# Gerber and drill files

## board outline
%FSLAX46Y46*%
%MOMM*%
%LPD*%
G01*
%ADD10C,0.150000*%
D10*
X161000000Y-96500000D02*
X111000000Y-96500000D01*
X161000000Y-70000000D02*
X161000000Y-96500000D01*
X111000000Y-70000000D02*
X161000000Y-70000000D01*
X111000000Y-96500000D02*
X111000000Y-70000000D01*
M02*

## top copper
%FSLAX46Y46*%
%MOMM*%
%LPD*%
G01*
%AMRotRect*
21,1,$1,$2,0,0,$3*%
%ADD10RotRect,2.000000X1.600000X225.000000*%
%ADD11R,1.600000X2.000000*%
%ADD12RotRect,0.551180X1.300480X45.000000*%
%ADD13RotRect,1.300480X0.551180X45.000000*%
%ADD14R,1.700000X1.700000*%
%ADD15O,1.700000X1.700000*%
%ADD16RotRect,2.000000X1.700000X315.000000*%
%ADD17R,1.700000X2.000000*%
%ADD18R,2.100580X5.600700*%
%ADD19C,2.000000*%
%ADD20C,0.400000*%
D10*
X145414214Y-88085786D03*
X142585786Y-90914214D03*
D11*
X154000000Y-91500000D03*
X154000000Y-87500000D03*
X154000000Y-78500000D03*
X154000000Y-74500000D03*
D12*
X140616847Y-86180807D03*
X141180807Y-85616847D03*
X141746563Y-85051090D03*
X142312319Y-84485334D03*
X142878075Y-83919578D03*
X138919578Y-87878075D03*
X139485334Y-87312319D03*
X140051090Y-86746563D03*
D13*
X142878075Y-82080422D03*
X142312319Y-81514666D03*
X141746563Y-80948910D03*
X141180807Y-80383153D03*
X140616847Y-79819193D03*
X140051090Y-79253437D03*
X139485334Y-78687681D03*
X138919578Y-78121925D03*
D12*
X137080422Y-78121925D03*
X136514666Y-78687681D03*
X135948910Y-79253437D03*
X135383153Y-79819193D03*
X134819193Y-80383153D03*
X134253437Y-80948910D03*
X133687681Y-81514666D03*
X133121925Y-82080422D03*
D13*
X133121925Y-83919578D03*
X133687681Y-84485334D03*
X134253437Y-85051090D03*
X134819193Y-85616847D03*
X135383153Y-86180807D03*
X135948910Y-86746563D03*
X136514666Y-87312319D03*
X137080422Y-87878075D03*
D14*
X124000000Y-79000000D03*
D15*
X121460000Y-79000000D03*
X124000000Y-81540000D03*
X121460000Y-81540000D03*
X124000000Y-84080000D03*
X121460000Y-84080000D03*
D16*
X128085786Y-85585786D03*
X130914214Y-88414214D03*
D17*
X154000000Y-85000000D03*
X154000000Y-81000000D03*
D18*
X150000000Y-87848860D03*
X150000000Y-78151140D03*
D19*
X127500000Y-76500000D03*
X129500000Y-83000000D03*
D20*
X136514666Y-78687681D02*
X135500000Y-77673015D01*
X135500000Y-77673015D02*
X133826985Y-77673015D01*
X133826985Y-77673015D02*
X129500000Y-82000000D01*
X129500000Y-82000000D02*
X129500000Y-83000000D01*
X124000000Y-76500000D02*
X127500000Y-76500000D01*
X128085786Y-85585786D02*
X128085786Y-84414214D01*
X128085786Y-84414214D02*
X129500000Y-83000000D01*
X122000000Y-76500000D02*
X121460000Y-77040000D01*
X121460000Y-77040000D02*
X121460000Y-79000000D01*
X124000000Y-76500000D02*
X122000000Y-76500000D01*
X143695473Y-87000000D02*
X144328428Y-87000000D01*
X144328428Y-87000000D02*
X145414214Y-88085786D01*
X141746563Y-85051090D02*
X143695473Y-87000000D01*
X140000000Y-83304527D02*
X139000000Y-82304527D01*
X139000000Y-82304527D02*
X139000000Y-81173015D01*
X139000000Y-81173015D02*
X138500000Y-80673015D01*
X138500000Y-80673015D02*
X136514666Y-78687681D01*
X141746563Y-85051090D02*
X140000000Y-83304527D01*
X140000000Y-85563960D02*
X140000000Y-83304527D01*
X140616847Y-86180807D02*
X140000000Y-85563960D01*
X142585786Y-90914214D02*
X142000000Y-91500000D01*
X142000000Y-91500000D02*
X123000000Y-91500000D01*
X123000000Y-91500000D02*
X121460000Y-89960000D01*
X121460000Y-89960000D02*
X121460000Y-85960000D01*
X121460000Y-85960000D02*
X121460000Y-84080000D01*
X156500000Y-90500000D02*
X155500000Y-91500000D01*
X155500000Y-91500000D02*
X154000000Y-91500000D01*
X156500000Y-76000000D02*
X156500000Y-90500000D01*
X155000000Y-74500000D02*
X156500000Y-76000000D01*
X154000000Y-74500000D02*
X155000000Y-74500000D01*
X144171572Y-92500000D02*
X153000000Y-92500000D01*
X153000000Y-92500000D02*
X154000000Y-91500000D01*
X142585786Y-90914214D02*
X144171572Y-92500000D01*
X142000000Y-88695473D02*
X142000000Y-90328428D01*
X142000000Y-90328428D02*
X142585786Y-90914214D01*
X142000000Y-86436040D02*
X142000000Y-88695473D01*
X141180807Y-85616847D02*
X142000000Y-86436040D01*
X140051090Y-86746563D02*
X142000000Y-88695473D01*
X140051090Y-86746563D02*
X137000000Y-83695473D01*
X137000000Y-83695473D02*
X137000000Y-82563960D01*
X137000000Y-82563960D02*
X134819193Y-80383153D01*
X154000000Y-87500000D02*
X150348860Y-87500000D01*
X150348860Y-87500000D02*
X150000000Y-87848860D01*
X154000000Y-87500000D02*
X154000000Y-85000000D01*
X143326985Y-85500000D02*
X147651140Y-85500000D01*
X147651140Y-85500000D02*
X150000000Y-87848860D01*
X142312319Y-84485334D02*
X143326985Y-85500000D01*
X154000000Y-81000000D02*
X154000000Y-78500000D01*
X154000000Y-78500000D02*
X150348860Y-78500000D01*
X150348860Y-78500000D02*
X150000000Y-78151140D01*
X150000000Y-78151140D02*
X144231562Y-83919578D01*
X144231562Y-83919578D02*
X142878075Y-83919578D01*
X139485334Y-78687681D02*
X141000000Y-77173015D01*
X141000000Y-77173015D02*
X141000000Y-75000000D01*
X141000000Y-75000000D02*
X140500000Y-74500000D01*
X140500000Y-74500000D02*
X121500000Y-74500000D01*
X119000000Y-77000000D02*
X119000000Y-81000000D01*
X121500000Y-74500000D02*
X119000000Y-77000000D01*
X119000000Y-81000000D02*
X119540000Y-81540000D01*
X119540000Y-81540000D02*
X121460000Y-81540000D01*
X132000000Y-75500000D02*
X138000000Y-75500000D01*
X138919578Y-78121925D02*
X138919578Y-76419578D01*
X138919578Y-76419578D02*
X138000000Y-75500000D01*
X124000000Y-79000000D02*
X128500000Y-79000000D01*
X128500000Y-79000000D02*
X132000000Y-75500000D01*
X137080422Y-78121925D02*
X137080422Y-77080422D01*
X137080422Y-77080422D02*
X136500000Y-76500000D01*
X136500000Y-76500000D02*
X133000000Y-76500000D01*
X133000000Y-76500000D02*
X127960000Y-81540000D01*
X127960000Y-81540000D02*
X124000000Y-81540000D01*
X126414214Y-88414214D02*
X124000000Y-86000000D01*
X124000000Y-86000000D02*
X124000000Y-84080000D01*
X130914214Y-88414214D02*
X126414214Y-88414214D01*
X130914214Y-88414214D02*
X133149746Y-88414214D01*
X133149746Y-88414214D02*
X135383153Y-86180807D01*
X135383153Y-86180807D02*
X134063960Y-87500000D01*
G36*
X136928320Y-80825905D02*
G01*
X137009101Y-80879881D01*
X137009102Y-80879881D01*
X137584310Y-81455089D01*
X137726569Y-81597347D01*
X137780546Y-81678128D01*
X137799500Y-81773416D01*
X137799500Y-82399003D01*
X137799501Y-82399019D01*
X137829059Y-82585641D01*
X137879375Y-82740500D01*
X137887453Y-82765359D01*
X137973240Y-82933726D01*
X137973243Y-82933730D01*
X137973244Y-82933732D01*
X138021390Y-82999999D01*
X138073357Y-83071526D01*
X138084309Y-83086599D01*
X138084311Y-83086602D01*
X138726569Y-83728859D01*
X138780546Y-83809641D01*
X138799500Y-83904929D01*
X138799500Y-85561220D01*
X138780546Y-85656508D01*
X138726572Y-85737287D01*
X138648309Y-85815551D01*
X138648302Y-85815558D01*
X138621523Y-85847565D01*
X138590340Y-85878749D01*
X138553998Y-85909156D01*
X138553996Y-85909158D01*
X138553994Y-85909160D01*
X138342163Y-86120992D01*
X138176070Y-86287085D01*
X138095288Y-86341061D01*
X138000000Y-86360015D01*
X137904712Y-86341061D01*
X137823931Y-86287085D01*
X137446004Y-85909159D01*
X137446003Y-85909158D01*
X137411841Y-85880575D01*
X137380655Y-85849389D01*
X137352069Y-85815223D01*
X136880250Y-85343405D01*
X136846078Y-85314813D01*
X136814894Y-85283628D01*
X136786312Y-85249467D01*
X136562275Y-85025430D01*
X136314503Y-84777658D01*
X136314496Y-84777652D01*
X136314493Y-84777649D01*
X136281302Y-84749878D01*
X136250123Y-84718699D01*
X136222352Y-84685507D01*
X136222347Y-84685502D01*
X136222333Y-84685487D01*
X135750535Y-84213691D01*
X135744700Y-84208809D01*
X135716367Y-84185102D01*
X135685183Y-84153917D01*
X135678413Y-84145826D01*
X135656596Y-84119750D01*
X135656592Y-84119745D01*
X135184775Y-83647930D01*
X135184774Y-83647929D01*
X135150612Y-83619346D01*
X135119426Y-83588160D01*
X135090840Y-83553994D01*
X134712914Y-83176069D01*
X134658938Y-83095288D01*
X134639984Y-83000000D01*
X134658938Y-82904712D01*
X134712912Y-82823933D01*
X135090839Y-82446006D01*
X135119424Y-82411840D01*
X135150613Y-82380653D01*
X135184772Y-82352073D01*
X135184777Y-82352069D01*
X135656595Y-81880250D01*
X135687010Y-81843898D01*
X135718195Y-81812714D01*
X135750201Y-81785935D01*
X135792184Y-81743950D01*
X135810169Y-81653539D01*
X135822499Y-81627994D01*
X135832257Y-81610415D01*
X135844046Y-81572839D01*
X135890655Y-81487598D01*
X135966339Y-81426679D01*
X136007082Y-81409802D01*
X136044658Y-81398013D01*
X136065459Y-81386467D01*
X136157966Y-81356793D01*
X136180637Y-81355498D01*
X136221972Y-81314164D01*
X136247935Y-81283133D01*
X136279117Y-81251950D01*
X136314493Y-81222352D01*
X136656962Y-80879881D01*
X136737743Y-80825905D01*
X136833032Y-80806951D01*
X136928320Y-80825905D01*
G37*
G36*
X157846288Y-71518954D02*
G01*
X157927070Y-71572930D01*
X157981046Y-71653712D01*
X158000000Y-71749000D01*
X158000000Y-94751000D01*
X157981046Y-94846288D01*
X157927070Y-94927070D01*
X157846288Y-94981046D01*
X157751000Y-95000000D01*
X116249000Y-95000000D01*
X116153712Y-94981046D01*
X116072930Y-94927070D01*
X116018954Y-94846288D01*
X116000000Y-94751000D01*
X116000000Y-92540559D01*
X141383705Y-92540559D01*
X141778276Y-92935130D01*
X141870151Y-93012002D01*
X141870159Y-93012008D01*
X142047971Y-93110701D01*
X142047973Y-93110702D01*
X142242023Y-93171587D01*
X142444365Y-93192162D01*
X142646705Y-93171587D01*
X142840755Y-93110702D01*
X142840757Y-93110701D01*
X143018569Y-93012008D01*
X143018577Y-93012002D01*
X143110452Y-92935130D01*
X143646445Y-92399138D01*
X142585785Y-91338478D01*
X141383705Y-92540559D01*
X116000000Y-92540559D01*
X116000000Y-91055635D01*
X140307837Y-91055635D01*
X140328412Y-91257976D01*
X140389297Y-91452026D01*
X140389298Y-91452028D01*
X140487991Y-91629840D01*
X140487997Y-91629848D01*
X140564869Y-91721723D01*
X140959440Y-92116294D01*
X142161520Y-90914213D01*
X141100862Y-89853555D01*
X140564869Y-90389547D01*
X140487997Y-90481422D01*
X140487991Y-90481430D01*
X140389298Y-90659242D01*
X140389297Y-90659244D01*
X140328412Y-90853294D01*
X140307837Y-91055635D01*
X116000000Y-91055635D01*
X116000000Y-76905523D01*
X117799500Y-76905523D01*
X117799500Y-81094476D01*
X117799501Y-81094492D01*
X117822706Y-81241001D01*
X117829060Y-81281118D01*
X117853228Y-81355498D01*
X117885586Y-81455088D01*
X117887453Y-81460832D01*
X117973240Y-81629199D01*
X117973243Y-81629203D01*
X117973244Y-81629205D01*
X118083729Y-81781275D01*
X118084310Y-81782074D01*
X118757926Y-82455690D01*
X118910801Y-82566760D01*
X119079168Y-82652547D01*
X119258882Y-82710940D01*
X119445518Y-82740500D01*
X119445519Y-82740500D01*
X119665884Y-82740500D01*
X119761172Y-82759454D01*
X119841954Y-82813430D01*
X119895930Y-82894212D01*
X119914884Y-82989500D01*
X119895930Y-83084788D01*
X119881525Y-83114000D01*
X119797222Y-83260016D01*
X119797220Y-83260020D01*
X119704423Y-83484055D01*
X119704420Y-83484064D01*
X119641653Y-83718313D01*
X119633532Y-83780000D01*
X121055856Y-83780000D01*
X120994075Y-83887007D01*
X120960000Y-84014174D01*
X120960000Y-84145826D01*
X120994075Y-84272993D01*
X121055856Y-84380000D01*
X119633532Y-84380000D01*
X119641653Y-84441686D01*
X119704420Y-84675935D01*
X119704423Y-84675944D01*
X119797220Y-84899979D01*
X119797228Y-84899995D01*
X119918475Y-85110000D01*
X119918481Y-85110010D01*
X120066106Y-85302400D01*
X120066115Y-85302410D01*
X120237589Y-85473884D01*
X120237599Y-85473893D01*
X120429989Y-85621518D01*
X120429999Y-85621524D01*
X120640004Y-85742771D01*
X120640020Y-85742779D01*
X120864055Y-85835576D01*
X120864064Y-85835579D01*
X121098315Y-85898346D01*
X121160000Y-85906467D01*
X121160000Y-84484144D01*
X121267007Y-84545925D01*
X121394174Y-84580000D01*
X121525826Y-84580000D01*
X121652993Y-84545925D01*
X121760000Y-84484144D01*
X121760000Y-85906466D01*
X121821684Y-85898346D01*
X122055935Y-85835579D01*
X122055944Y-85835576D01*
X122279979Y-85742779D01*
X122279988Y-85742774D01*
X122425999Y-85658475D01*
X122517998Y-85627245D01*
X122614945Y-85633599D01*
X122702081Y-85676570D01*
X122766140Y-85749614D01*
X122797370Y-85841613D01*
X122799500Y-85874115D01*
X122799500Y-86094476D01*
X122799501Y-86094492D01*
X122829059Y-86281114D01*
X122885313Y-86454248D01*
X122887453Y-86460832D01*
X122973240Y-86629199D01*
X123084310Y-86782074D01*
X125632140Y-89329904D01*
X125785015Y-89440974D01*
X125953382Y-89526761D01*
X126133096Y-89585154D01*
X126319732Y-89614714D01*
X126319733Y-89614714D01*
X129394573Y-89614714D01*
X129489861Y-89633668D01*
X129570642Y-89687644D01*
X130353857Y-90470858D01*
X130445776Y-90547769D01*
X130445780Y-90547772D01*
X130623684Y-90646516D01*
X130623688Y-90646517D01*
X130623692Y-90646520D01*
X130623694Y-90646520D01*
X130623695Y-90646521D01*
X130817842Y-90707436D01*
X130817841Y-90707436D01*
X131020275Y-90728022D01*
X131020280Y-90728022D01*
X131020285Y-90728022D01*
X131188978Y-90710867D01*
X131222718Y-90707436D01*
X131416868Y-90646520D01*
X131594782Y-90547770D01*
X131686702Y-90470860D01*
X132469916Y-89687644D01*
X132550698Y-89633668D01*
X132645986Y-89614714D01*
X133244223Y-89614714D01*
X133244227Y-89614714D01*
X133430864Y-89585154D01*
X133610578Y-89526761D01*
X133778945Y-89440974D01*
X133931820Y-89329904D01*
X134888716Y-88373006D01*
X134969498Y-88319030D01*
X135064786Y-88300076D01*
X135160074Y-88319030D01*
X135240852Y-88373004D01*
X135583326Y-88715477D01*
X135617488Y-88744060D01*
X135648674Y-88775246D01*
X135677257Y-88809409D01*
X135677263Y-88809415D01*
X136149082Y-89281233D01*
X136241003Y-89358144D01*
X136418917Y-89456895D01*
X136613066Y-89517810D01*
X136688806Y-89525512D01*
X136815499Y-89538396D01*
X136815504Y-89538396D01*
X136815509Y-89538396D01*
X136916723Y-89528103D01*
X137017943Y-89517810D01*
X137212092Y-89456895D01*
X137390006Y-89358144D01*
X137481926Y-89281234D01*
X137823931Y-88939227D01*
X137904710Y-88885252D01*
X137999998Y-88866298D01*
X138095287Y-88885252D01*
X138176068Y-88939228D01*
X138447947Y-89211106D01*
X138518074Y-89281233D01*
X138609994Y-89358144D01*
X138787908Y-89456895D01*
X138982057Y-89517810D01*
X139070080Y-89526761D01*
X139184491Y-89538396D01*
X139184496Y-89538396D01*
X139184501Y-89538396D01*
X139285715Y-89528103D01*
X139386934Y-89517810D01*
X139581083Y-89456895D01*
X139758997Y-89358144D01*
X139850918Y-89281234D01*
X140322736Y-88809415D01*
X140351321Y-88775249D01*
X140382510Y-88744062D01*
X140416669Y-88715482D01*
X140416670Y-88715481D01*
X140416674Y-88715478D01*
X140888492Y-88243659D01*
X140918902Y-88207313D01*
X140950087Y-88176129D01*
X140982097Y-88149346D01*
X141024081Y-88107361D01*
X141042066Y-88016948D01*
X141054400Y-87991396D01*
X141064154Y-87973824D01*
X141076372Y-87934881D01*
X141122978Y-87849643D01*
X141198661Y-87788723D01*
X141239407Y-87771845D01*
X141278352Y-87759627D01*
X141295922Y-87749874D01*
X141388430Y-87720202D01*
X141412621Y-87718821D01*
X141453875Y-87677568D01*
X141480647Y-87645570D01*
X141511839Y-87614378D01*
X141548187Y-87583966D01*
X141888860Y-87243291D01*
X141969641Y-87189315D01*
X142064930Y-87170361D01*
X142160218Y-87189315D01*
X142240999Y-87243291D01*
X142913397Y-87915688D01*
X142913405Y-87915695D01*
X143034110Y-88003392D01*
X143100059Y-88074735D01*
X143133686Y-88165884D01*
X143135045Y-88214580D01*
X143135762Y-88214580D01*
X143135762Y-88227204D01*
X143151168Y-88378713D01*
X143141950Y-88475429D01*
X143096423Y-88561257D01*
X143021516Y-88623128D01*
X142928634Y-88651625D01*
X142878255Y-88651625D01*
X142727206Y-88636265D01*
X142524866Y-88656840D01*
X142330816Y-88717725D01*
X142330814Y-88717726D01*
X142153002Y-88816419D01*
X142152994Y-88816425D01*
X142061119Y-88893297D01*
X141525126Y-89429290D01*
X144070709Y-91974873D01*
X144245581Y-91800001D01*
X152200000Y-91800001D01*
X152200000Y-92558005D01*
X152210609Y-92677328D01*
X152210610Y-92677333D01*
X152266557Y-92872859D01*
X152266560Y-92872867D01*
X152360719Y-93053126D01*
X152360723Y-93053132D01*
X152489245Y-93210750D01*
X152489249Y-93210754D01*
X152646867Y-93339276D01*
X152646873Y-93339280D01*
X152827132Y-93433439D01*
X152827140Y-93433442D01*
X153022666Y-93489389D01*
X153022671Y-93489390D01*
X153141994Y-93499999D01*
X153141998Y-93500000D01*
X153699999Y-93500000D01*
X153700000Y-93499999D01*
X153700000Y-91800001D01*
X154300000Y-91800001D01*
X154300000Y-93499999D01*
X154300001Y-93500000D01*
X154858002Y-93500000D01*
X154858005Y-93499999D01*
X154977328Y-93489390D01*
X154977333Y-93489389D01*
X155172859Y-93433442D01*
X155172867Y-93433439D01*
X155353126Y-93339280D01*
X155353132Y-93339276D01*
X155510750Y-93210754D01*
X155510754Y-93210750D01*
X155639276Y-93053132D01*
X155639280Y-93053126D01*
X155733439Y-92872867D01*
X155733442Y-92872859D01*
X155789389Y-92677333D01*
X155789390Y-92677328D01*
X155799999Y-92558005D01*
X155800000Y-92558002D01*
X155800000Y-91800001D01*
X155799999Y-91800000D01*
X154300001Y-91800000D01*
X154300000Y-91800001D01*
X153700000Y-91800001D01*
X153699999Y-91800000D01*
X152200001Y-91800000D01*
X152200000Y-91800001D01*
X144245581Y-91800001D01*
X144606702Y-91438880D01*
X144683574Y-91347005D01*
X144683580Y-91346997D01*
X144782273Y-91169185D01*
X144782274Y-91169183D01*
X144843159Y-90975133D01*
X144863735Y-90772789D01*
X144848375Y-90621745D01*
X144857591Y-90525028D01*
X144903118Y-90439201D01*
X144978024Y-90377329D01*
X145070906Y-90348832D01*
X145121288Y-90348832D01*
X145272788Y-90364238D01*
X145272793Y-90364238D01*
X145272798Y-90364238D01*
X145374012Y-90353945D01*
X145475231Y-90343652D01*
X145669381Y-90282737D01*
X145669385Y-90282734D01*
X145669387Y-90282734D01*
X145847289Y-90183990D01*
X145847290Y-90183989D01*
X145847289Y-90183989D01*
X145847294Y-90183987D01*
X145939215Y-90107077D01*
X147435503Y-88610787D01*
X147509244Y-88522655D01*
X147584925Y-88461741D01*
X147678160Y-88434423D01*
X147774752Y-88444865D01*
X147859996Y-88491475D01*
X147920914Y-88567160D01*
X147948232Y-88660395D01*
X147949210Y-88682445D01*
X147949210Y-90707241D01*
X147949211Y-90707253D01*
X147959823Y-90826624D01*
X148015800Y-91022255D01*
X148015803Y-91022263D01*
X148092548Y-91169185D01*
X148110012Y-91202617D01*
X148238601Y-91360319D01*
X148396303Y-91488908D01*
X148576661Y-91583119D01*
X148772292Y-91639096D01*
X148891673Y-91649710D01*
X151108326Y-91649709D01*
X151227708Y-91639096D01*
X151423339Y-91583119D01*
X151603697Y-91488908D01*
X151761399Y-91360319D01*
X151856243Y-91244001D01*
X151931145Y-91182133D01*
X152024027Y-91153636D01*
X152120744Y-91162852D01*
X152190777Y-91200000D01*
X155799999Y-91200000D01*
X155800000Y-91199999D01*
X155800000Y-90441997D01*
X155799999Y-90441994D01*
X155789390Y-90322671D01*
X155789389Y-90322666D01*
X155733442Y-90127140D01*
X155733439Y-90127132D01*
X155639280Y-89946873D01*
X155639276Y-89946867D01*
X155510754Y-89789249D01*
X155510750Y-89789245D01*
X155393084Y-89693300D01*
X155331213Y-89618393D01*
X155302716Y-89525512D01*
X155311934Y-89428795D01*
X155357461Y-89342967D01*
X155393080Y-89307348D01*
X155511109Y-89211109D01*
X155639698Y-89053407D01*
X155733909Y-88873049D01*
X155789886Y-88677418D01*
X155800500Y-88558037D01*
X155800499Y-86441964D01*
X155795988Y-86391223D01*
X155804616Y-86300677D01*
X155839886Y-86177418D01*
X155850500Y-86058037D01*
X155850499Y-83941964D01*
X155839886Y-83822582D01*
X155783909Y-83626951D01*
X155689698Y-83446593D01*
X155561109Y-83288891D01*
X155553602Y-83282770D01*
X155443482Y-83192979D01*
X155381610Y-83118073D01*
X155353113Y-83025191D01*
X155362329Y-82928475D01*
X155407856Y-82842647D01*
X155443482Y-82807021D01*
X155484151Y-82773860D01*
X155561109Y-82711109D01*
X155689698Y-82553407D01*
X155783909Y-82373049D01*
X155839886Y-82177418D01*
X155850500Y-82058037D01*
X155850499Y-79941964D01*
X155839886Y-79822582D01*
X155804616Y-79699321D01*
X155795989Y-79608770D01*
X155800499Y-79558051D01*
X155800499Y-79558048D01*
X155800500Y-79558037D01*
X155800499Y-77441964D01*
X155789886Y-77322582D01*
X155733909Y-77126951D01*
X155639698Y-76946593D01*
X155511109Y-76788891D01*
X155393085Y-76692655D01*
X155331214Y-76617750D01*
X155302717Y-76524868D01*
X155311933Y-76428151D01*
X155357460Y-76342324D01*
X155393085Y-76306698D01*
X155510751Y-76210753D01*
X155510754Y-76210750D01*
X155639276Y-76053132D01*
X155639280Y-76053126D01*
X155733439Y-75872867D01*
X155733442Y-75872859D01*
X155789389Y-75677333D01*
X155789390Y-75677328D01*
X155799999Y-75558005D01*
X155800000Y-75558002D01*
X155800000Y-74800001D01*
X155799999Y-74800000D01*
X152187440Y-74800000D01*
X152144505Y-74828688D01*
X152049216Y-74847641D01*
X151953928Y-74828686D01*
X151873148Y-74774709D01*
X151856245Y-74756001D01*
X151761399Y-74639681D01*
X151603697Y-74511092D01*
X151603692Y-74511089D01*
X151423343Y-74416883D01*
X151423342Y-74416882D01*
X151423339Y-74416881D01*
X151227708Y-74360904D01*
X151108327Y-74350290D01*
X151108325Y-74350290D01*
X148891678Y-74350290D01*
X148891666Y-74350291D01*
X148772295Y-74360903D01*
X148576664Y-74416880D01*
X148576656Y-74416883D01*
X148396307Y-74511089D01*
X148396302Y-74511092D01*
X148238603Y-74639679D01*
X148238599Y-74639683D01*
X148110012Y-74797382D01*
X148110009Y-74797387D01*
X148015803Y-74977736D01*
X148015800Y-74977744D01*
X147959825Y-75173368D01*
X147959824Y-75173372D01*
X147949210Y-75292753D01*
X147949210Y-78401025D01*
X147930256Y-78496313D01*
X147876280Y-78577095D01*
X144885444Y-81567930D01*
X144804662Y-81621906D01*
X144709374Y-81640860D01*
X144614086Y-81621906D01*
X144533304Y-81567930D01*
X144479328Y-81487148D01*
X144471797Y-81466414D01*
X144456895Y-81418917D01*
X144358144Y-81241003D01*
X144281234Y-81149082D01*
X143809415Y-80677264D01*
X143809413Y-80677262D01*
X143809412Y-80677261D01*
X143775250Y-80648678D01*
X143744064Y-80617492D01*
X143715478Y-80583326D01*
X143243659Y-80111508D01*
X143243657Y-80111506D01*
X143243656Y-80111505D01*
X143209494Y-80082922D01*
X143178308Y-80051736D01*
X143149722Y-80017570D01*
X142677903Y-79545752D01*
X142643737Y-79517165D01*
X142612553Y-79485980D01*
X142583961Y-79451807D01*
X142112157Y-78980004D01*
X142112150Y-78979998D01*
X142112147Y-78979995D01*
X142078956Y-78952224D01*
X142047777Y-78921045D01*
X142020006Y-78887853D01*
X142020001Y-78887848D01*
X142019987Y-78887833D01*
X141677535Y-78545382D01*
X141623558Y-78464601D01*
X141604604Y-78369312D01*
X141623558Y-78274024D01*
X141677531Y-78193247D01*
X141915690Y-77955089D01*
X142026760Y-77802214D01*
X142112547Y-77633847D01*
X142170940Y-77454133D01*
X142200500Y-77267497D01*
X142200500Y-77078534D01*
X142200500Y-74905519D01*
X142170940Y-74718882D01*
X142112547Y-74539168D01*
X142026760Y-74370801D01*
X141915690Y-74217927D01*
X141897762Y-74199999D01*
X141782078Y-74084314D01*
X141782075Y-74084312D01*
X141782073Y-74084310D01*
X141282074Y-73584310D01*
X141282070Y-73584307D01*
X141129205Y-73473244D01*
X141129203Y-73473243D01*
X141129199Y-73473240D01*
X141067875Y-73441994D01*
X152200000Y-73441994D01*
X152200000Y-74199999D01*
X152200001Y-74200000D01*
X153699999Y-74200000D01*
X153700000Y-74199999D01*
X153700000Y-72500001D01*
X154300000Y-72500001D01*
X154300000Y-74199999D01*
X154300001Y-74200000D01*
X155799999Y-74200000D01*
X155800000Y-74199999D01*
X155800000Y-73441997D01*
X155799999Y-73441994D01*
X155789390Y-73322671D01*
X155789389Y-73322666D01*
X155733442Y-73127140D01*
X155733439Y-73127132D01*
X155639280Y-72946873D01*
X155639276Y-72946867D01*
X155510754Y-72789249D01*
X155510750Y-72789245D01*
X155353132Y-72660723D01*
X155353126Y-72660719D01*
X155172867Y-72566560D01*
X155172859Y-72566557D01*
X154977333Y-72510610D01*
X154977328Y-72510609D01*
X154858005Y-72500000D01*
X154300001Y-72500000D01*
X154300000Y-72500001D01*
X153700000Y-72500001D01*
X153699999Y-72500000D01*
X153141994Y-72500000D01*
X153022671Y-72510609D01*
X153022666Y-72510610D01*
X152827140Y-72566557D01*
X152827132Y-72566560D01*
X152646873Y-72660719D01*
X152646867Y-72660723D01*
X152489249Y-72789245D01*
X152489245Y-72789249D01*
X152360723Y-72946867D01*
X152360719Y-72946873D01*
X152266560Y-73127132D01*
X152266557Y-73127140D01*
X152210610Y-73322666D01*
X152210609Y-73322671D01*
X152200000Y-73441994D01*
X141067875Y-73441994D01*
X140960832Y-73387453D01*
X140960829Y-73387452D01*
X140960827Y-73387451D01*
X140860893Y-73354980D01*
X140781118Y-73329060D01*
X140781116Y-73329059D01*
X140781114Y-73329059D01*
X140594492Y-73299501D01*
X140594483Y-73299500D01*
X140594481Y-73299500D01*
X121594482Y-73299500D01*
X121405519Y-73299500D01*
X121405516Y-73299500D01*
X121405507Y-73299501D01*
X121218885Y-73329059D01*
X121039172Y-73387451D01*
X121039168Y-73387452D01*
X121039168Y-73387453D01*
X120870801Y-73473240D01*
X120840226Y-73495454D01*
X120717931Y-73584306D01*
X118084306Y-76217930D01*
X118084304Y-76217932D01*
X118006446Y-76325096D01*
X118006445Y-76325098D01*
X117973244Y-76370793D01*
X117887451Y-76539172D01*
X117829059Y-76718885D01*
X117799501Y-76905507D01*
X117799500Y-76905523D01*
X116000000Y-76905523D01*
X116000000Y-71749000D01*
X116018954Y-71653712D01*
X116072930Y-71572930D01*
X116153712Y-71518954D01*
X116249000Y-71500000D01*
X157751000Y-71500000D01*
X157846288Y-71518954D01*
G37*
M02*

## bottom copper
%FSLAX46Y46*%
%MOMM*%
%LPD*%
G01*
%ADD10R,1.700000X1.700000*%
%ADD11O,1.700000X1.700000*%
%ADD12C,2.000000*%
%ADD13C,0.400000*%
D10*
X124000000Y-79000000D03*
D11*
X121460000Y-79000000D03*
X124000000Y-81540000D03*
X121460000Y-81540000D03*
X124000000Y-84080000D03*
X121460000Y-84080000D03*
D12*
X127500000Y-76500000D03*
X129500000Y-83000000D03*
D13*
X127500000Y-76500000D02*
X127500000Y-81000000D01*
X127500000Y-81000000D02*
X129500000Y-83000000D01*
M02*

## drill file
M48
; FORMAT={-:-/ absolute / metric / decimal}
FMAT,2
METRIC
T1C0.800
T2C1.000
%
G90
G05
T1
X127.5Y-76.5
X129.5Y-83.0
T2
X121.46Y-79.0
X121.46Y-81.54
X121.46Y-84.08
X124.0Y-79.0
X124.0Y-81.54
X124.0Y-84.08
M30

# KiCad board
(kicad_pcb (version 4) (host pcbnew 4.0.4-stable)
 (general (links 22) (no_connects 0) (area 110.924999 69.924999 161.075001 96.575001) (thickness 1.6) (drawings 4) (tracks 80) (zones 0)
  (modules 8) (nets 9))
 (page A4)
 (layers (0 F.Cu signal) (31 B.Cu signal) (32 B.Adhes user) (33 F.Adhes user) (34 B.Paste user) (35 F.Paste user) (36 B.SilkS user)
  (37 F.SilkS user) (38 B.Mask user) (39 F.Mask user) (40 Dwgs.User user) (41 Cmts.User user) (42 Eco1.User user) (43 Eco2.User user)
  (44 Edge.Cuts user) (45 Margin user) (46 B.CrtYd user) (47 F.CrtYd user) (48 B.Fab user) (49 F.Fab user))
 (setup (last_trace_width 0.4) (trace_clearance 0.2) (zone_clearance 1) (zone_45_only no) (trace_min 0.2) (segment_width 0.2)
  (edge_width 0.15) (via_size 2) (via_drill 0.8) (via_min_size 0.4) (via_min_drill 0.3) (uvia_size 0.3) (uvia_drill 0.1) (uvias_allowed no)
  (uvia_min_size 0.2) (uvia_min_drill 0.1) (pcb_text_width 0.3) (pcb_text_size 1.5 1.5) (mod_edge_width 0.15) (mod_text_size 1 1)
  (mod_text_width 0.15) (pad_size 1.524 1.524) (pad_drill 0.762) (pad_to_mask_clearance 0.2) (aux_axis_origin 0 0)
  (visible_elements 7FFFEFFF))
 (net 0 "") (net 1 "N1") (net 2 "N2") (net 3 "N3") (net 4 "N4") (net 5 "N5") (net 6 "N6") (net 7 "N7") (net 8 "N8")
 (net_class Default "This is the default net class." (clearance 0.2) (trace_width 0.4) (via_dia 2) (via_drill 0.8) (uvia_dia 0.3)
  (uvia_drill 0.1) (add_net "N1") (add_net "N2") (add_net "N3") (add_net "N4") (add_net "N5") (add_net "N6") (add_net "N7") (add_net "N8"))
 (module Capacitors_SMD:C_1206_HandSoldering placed (layer F.Cu) (at 144 89.5 225)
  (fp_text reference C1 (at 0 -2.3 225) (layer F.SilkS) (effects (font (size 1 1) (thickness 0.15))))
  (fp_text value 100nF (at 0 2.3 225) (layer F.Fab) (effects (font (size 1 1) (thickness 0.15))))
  (pad 1 smd rect (at -2 0 225) (size 2 1.6) (layers F.Cu F.Paste F.Mask) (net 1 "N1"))
  (pad 2 smd rect (at 2 0 225) (size 2 1.6) (layers F.Cu F.Paste F.Mask) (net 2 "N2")))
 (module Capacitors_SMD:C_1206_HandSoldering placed (layer F.Cu) (at 154 89.5 90)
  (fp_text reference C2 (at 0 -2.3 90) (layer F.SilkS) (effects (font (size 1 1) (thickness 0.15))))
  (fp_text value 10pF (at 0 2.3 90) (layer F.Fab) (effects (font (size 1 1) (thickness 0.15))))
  (pad 1 smd rect (at -2 0 90) (size 2 1.6) (layers F.Cu F.Paste F.Mask) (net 2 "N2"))
  (pad 2 smd rect (at 2 0 90) (size 2 1.6) (layers F.Cu F.Paste F.Mask) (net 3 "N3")))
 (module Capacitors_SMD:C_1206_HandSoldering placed (layer F.Cu) (at 154 76.5 90)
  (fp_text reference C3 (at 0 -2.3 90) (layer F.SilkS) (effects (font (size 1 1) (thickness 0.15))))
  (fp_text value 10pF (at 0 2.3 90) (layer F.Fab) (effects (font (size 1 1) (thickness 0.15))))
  (pad 1 smd rect (at -2 0 90) (size 2 1.6) (layers F.Cu F.Paste F.Mask) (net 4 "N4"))
  (pad 2 smd rect (at 2 0 90) (size 2 1.6) (layers F.Cu F.Paste F.Mask) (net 2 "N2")))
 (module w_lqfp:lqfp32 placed (layer F.Cu) (at 138 83 45)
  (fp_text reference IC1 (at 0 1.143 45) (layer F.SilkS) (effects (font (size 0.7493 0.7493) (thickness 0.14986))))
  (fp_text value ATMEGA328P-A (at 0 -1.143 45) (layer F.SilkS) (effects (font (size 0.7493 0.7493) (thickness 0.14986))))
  (pad 4 smd rect (at -0.39878 4.09956 45) (size 0.55118 1.30048) (layers F.Cu F.Paste F.Mask) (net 1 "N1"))
  (pad 5 smd rect (at 0.39878 4.09956 45) (size 0.55118 1.30048) (layers F.Cu F.Paste F.Mask) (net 2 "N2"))
  (pad 6 smd rect (at 1.19888 4.09956 45) (size 0.55118 1.30048) (layers F.Cu F.Paste F.Mask) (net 1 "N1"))
  (pad 7 smd rect (at 1.99898 4.09956 45) (size 0.55118 1.30048) (layers F.Cu F.Paste F.Mask) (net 3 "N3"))
  (pad 8 smd rect (at 2.79908 4.09956 45) (size 0.55118 1.30048) (layers F.Cu F.Paste F.Mask) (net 4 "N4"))
  (pad 1 smd rect (at -2.79908 4.09956 45) (size 0.55118 1.30048) (layers F.Cu F.Paste F.Mask))
  (pad 2 smd rect (at -1.99898 4.09956 45) (size 0.55118 1.30048) (layers F.Cu F.Paste F.Mask))
  (pad 3 smd rect (at -1.19888 4.09956 45) (size 0.55118 1.30048) (layers F.Cu F.Paste F.Mask) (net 2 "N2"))
  (pad 9 smd rect (at 4.09956 2.79908 45) (size 1.30048 0.55118) (layers F.Cu F.Paste F.Mask))
  (pad 10 smd rect (at 4.09956 1.99898 45) (size 1.30048 0.55118) (layers F.Cu F.Paste F.Mask))
  (pad 11 smd rect (at 4.09956 1.19888 45) (size 1.30048 0.55118) (layers F.Cu F.Paste F.Mask))
  (pad 12 smd rect (at 4.09956 0.39878 45) (size 1.30048 0.55118) (layers F.Cu F.Paste F.Mask))
  (pad 13 smd rect (at 4.09956 -0.39878 45) (size 1.30048 0.55118) (layers F.Cu F.Paste F.Mask))
  (pad 14 smd rect (at 4.09956 -1.19888 45) (size 1.30048 0.55118) (layers F.Cu F.Paste F.Mask))
  (pad 15 smd rect (at 4.09956 -1.99898 45) (size 1.30048 0.55118) (layers F.Cu F.Paste F.Mask) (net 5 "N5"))
  (pad 16 smd rect (at 4.09956 -2.79908 45) (size 1.30048 0.55118) (layers F.Cu F.Paste F.Mask) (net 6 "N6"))
  (pad 17 smd rect (at 2.79908 -4.09956 45) (size 0.55118 1.30048) (layers F.Cu F.Paste F.Mask) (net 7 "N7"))
  (pad 18 smd rect (at 1.99898 -4.09956 45) (size 0.55118 1.30048) (layers F.Cu F.Paste F.Mask) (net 1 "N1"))
  (pad 19 smd rect (at 1.19888 -4.09956 45) (size 0.55118 1.30048) (layers F.Cu F.Paste F.Mask))
  (pad 20 smd rect (at 0.39878 -4.09956 45) (size 0.55118 1.30048) (layers F.Cu F.Paste F.Mask))
  (pad 21 smd rect (at -0.39878 -4.09956 45) (size 0.55118 1.30048) (layers F.Cu F.Paste F.Mask) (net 2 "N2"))
  (pad 22 smd rect (at -1.19888 -4.09956 45) (size 0.55118 1.30048) (layers F.Cu F.Paste F.Mask))
  (pad 23 smd rect (at -1.99898 -4.09956 45) (size 0.55118 1.30048) (layers F.Cu F.Paste F.Mask))
  (pad 24 smd rect (at -2.79908 -4.09956 45) (size 0.55118 1.30048) (layers F.Cu F.Paste F.Mask))
  (pad 25 smd rect (at -4.09956 -2.79908 45) (size 1.30048 0.55118) (layers F.Cu F.Paste F.Mask))
  (pad 26 smd rect (at -4.09956 -1.99898 45) (size 1.30048 0.55118) (layers F.Cu F.Paste F.Mask))
  (pad 27 smd rect (at -4.09956 -1.19888 45) (size 1.30048 0.55118) (layers F.Cu F.Paste F.Mask))
  (pad 28 smd rect (at -4.09956 -0.39878 45) (size 1.30048 0.55118) (layers F.Cu F.Paste F.Mask))
  (pad 29 smd rect (at -4.09956 0.39878 45) (size 1.30048 0.55118) (layers F.Cu F.Paste F.Mask) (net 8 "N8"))
  (pad 30 smd rect (at -4.09956 1.19888 45) (size 1.30048 0.55118) (layers F.Cu F.Paste F.Mask))
  (pad 31 smd rect (at -4.09956 1.99898 45) (size 1.30048 0.55118) (layers F.Cu F.Paste F.Mask))
  (pad 32 smd rect (at -4.09956 2.79908 45) (size 1.30048 0.55118) (layers F.Cu F.Paste F.Mask)))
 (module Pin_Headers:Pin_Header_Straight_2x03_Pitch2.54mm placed (layer B.Cu) (at 124 79 180)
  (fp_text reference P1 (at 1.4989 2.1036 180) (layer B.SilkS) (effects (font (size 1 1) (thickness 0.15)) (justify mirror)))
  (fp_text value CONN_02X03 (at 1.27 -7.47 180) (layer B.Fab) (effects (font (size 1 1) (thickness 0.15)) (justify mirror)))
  (pad 1 thru_hole rect (at 0 0 180) (size 1.7 1.7) (drill 1) (layers *.Cu *.Mask) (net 6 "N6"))
  (pad 2 thru_hole oval (at 2.54 0 180) (size 1.7 1.7) (drill 1) (layers *.Cu *.Mask) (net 1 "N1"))
  (pad 3 thru_hole oval (at 0 -2.54 180) (size 1.7 1.7) (drill 1) (layers *.Cu *.Mask) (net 7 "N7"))
  (pad 4 thru_hole oval (at 2.54 -2.54 180) (size 1.7 1.7) (drill 1) (layers *.Cu *.Mask) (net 5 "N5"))
  (pad 5 thru_hole oval (at 0 -5.08 180) (size 1.7 1.7) (drill 1) (layers *.Cu *.Mask) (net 8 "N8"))
  (pad 6 thru_hole oval (at 2.54 -5.08 180) (size 1.7 1.7) (drill 1) (layers *.Cu *.Mask) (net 2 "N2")))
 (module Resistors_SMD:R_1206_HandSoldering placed (layer F.Cu) (at 129.5 87 315)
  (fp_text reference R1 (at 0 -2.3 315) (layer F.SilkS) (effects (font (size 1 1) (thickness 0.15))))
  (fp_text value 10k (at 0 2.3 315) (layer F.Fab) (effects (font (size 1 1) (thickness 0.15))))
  (pad 1 smd rect (at -2 0 315) (size 2 1.7) (layers F.Cu F.Paste F.Mask) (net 1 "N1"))
  (pad 2 smd rect (at 2 0 315) (size 2 1.7) (layers F.Cu F.Paste F.Mask) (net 8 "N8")))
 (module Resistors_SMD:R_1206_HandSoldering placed (layer F.Cu) (at 154 83 90)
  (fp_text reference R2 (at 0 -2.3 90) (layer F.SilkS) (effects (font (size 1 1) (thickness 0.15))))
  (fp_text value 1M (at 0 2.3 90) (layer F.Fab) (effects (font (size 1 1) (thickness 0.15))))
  (pad 1 smd rect (at -2 0 90) (size 2 1.7) (layers F.Cu F.Paste F.Mask) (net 3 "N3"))
  (pad 2 smd rect (at 2 0 90) (size 2 1.7) (layers F.Cu F.Paste F.Mask) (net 4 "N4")))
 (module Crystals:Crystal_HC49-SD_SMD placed (layer F.Cu) (at 150 83 90)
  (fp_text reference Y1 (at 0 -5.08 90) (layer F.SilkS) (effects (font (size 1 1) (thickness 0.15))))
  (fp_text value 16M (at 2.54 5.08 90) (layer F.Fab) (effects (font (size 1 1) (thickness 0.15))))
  (pad 1 smd rect (at -4.84886 0 90) (size 5.6007 2.10058) (layers F.Cu F.Paste F.Mask) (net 3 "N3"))
  (pad 2 smd rect (at 4.84886 0 90) (size 5.6007 2.10058) (layers F.Cu F.Paste F.Mask) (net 4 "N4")))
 (gr_line (start 161 96.5) (end 111 96.5) (angle 90) (layer Edge.Cuts) (width 0.15))
 (gr_line (start 161 70) (end 161 96.5) (angle 90) (layer Edge.Cuts) (width 0.15))
 (gr_line (start 111 70) (end 161 70) (angle 90) (layer Edge.Cuts) (width 0.15))
 (gr_line (start 111 96.5) (end 111 70) (angle 90) (layer Edge.Cuts) (width 0.15))
 (segment (start 136.514666 78.687681) (end 135.5 77.673015) (width 0.4) (layer F.Cu) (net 1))
 (segment (start 135.5 77.673015) (end 133.826985 77.673015) (width 0.4) (layer F.Cu) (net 1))
 (segment (start 133.826985 77.673015) (end 129.5 82) (width 0.4) (layer F.Cu) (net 1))
 (segment (start 129.5 82) (end 129.5 83) (width 0.4) (layer F.Cu) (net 1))
 (segment (start 127.5 76.5) (end 127.5 81) (width 0.4) (layer B.Cu) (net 1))
 (segment (start 127.5 81) (end 129.5 83) (width 0.4) (layer B.Cu) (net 1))
 (segment (start 124 76.5) (end 127.5 76.5) (width 0.4) (layer F.Cu) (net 1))
 (via (at 127.5 76.5) (size 2) (drill 0.8) (layers F.Cu B.Cu) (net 1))
 (via (at 129.5 83) (size 2) (drill 0.8) (layers F.Cu B.Cu) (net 1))
 (segment (start 128.085786 85.585786) (end 128.085786 84.414214) (width 0.4) (layer F.Cu) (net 1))
 (segment (start 128.085786 84.414214) (end 129.5 83) (width 0.4) (layer F.Cu) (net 1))
 (segment (start 122 76.5) (end 121.46 77.04) (width 0.4) (layer F.Cu) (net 1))
 (segment (start 121.46 77.04) (end 121.46 79) (width 0.4) (layer F.Cu) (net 1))
 (segment (start 124 76.5) (end 122 76.5) (width 0.4) (layer F.Cu) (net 1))
 (segment (start 143.695473 87) (end 144.328428 87) (width 0.4) (layer F.Cu) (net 1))
 (segment (start 144.328428 87) (end 145.414214 88.085786) (width 0.4) (layer F.Cu) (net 1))
 (segment (start 141.746563 85.05109) (end 143.695473 87) (width 0.4) (layer F.Cu) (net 1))
 (segment (start 140 83.304527) (end 139 82.304527) (width 0.4) (layer F.Cu) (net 1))
 (segment (start 139 82.304527) (end 139 81.173015) (width 0.4) (layer F.Cu) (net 1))
 (segment (start 139 81.173015) (end 138.5 80.673015) (width 0.4) (layer F.Cu) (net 1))
 (segment (start 138.5 80.673015) (end 136.514666 78.687681) (width 0.4) (layer F.Cu) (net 1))
 (segment (start 141.746563 85.05109) (end 140 83.304527) (width 0.4) (layer F.Cu) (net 1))
 (segment (start 140 85.56396) (end 140 83.304527) (width 0.4) (layer F.Cu) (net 1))
 (segment (start 140.616847 86.180807) (end 140 85.56396) (width 0.4) (layer F.Cu) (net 1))
 (segment (start 142.585786 90.914214) (end 142 91.5) (width 0.4) (layer F.Cu) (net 2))
 (segment (start 142 91.5) (end 123 91.5) (width 0.4) (layer F.Cu) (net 2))
 (segment (start 123 91.5) (end 121.46 89.96) (width 0.4) (layer F.Cu) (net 2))
 (segment (start 121.46 89.96) (end 121.46 85.96) (width 0.4) (layer F.Cu) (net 2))
 (segment (start 121.46 85.96) (end 121.46 84.08) (width 0.4) (layer F.Cu) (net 2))
 (segment (start 156.5 90.5) (end 155.5 91.5) (width 0.4) (layer F.Cu) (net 2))
 (segment (start 155.5 91.5) (end 154 91.5) (width 0.4) (layer F.Cu) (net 2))
 (segment (start 156.5 76) (end 156.5 90.5) (width 0.4) (layer F.Cu) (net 2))
 (segment (start 155 74.5) (end 156.5 76) (width 0.4) (layer F.Cu) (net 2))
 (segment (start 154 74.5) (end 155 74.5) (width 0.4) (layer F.Cu) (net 2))
 (segment (start 144.171572 92.5) (end 153 92.5) (width 0.4) (layer F.Cu) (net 2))
 (segment (start 153 92.5) (end 154 91.5) (width 0.4) (layer F.Cu) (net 2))
 (segment (start 142.585786 90.914214) (end 144.171572 92.5) (width 0.4) (layer F.Cu) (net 2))
 (segment (start 142 88.695473) (end 142 90.328428) (width 0.4) (layer F.Cu) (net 2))
 (segment (start 142 90.328428) (end 142.585786 90.914214) (width 0.4) (layer F.Cu) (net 2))
 (segment (start 142 86.43604) (end 142 88.695473) (width 0.4) (layer F.Cu) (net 2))
 (segment (start 141.180807 85.616847) (end 142 86.43604) (width 0.4) (layer F.Cu) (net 2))
 (segment (start 140.05109 86.746563) (end 142 88.695473) (width 0.4) (layer F.Cu) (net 2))
 (segment (start 140.05109 86.746563) (end 137 83.695473) (width 0.4) (layer F.Cu) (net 2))
 (segment (start 137 83.695473) (end 137 82.56396) (width 0.4) (layer F.Cu) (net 2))
 (segment (start 137 82.56396) (end 134.819193 80.383153) (width 0.4) (layer F.Cu) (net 2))
 (segment (start 154 87.5) (end 150.34886 87.5) (width 0.4) (layer F.Cu) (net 3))
 (segment (start 150.34886 87.5) (end 150 87.84886) (width 0.4) (layer F.Cu) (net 3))
 (segment (start 154 87.5) (end 154 85) (width 0.4) (layer F.Cu) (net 3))
 (segment (start 143.326985 85.5) (end 147.65114 85.5) (width 0.4) (layer F.Cu) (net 3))
 (segment (start 147.65114 85.5) (end 150 87.84886) (width 0.4) (layer F.Cu) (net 3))
 (segment (start 142.312319 84.485334) (end 143.326985 85.5) (width 0.4) (layer F.Cu) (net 3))
 (segment (start 154 81) (end 154 78.5) (width 0.4) (layer F.Cu) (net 4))
 (segment (start 154 78.5) (end 150.34886 78.5) (width 0.4) (layer F.Cu) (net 4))
 (segment (start 150.34886 78.5) (end 150 78.15114) (width 0.4) (layer F.Cu) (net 4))
 (segment (start 150 78.15114) (end 144.231562 83.919578) (width 0.4) (layer F.Cu) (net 4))
 (segment (start 144.231562 83.919578) (end 142.878075 83.919578) (width 0.4) (layer F.Cu) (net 4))
 (segment (start 139.485334 78.687681) (end 141 77.173015) (width 0.4) (layer F.Cu) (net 5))
 (segment (start 141 77.173015) (end 141 75) (width 0.4) (layer F.Cu) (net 5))
 (segment (start 141 75) (end 140.5 74.5) (width 0.4) (layer F.Cu) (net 5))
 (segment (start 140.5 74.5) (end 121.5 74.5) (width 0.4) (layer F.Cu) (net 5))
 (segment (start 119 77) (end 119 81) (width 0.4) (layer F.Cu) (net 5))
 (segment (start 121.5 74.5) (end 119 77) (width 0.4) (layer F.Cu) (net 5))
 (segment (start 119 81) (end 119.54 81.54) (width 0.4) (layer F.Cu) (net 5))
 (segment (start 119.54 81.54) (end 121.46 81.54) (width 0.4) (layer F.Cu) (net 5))
 (segment (start 132 75.5) (end 138 75.5) (width 0.4) (layer F.Cu) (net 6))
 (segment (start 138.919578 78.121925) (end 138.919578 76.419578) (width 0.4) (layer F.Cu) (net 6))
 (segment (start 138.919578 76.419578) (end 138 75.5) (width 0.4) (layer F.Cu) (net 6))
 (segment (start 124 79) (end 128.5 79) (width 0.4) (layer F.Cu) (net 6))
 (segment (start 128.5 79) (end 132 75.5) (width 0.4) (layer F.Cu) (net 6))
 (segment (start 137.080422 78.121925) (end 137.080422 77.080422) (width 0.4) (layer F.Cu) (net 7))
 (segment (start 137.080422 77.080422) (end 136.5 76.5) (width 0.4) (layer F.Cu) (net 7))
 (segment (start 136.5 76.5) (end 133 76.5) (width 0.4) (layer F.Cu) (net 7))
 (segment (start 133 76.5) (end 127.96 81.54) (width 0.4) (layer F.Cu) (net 7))
 (segment (start 127.96 81.54) (end 124 81.54) (width 0.4) (layer F.Cu) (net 7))
 (segment (start 126.414214 88.414214) (end 124 86) (width 0.4) (layer F.Cu) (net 8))
 (segment (start 124 86) (end 124 84.08) (width 0.4) (layer F.Cu) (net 8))
 (segment (start 130.914214 88.414214) (end 126.414214 88.414214) (width 0.4) (layer F.Cu) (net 8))
 (segment (start 130.914214 88.414214) (end 133.149746 88.414214) (width 0.4) (layer F.Cu) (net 8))
 (segment (start 133.149746 88.414214) (end 135.383153 86.180807) (width 0.4) (layer F.Cu) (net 8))
 (segment (start 135.383153 86.180807) (end 134.06396 87.5) (width 0.4) (layer F.Cu) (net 8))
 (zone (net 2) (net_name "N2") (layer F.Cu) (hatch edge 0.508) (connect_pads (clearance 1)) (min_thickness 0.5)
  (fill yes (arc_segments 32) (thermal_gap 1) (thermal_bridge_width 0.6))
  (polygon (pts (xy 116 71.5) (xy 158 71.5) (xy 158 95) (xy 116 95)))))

